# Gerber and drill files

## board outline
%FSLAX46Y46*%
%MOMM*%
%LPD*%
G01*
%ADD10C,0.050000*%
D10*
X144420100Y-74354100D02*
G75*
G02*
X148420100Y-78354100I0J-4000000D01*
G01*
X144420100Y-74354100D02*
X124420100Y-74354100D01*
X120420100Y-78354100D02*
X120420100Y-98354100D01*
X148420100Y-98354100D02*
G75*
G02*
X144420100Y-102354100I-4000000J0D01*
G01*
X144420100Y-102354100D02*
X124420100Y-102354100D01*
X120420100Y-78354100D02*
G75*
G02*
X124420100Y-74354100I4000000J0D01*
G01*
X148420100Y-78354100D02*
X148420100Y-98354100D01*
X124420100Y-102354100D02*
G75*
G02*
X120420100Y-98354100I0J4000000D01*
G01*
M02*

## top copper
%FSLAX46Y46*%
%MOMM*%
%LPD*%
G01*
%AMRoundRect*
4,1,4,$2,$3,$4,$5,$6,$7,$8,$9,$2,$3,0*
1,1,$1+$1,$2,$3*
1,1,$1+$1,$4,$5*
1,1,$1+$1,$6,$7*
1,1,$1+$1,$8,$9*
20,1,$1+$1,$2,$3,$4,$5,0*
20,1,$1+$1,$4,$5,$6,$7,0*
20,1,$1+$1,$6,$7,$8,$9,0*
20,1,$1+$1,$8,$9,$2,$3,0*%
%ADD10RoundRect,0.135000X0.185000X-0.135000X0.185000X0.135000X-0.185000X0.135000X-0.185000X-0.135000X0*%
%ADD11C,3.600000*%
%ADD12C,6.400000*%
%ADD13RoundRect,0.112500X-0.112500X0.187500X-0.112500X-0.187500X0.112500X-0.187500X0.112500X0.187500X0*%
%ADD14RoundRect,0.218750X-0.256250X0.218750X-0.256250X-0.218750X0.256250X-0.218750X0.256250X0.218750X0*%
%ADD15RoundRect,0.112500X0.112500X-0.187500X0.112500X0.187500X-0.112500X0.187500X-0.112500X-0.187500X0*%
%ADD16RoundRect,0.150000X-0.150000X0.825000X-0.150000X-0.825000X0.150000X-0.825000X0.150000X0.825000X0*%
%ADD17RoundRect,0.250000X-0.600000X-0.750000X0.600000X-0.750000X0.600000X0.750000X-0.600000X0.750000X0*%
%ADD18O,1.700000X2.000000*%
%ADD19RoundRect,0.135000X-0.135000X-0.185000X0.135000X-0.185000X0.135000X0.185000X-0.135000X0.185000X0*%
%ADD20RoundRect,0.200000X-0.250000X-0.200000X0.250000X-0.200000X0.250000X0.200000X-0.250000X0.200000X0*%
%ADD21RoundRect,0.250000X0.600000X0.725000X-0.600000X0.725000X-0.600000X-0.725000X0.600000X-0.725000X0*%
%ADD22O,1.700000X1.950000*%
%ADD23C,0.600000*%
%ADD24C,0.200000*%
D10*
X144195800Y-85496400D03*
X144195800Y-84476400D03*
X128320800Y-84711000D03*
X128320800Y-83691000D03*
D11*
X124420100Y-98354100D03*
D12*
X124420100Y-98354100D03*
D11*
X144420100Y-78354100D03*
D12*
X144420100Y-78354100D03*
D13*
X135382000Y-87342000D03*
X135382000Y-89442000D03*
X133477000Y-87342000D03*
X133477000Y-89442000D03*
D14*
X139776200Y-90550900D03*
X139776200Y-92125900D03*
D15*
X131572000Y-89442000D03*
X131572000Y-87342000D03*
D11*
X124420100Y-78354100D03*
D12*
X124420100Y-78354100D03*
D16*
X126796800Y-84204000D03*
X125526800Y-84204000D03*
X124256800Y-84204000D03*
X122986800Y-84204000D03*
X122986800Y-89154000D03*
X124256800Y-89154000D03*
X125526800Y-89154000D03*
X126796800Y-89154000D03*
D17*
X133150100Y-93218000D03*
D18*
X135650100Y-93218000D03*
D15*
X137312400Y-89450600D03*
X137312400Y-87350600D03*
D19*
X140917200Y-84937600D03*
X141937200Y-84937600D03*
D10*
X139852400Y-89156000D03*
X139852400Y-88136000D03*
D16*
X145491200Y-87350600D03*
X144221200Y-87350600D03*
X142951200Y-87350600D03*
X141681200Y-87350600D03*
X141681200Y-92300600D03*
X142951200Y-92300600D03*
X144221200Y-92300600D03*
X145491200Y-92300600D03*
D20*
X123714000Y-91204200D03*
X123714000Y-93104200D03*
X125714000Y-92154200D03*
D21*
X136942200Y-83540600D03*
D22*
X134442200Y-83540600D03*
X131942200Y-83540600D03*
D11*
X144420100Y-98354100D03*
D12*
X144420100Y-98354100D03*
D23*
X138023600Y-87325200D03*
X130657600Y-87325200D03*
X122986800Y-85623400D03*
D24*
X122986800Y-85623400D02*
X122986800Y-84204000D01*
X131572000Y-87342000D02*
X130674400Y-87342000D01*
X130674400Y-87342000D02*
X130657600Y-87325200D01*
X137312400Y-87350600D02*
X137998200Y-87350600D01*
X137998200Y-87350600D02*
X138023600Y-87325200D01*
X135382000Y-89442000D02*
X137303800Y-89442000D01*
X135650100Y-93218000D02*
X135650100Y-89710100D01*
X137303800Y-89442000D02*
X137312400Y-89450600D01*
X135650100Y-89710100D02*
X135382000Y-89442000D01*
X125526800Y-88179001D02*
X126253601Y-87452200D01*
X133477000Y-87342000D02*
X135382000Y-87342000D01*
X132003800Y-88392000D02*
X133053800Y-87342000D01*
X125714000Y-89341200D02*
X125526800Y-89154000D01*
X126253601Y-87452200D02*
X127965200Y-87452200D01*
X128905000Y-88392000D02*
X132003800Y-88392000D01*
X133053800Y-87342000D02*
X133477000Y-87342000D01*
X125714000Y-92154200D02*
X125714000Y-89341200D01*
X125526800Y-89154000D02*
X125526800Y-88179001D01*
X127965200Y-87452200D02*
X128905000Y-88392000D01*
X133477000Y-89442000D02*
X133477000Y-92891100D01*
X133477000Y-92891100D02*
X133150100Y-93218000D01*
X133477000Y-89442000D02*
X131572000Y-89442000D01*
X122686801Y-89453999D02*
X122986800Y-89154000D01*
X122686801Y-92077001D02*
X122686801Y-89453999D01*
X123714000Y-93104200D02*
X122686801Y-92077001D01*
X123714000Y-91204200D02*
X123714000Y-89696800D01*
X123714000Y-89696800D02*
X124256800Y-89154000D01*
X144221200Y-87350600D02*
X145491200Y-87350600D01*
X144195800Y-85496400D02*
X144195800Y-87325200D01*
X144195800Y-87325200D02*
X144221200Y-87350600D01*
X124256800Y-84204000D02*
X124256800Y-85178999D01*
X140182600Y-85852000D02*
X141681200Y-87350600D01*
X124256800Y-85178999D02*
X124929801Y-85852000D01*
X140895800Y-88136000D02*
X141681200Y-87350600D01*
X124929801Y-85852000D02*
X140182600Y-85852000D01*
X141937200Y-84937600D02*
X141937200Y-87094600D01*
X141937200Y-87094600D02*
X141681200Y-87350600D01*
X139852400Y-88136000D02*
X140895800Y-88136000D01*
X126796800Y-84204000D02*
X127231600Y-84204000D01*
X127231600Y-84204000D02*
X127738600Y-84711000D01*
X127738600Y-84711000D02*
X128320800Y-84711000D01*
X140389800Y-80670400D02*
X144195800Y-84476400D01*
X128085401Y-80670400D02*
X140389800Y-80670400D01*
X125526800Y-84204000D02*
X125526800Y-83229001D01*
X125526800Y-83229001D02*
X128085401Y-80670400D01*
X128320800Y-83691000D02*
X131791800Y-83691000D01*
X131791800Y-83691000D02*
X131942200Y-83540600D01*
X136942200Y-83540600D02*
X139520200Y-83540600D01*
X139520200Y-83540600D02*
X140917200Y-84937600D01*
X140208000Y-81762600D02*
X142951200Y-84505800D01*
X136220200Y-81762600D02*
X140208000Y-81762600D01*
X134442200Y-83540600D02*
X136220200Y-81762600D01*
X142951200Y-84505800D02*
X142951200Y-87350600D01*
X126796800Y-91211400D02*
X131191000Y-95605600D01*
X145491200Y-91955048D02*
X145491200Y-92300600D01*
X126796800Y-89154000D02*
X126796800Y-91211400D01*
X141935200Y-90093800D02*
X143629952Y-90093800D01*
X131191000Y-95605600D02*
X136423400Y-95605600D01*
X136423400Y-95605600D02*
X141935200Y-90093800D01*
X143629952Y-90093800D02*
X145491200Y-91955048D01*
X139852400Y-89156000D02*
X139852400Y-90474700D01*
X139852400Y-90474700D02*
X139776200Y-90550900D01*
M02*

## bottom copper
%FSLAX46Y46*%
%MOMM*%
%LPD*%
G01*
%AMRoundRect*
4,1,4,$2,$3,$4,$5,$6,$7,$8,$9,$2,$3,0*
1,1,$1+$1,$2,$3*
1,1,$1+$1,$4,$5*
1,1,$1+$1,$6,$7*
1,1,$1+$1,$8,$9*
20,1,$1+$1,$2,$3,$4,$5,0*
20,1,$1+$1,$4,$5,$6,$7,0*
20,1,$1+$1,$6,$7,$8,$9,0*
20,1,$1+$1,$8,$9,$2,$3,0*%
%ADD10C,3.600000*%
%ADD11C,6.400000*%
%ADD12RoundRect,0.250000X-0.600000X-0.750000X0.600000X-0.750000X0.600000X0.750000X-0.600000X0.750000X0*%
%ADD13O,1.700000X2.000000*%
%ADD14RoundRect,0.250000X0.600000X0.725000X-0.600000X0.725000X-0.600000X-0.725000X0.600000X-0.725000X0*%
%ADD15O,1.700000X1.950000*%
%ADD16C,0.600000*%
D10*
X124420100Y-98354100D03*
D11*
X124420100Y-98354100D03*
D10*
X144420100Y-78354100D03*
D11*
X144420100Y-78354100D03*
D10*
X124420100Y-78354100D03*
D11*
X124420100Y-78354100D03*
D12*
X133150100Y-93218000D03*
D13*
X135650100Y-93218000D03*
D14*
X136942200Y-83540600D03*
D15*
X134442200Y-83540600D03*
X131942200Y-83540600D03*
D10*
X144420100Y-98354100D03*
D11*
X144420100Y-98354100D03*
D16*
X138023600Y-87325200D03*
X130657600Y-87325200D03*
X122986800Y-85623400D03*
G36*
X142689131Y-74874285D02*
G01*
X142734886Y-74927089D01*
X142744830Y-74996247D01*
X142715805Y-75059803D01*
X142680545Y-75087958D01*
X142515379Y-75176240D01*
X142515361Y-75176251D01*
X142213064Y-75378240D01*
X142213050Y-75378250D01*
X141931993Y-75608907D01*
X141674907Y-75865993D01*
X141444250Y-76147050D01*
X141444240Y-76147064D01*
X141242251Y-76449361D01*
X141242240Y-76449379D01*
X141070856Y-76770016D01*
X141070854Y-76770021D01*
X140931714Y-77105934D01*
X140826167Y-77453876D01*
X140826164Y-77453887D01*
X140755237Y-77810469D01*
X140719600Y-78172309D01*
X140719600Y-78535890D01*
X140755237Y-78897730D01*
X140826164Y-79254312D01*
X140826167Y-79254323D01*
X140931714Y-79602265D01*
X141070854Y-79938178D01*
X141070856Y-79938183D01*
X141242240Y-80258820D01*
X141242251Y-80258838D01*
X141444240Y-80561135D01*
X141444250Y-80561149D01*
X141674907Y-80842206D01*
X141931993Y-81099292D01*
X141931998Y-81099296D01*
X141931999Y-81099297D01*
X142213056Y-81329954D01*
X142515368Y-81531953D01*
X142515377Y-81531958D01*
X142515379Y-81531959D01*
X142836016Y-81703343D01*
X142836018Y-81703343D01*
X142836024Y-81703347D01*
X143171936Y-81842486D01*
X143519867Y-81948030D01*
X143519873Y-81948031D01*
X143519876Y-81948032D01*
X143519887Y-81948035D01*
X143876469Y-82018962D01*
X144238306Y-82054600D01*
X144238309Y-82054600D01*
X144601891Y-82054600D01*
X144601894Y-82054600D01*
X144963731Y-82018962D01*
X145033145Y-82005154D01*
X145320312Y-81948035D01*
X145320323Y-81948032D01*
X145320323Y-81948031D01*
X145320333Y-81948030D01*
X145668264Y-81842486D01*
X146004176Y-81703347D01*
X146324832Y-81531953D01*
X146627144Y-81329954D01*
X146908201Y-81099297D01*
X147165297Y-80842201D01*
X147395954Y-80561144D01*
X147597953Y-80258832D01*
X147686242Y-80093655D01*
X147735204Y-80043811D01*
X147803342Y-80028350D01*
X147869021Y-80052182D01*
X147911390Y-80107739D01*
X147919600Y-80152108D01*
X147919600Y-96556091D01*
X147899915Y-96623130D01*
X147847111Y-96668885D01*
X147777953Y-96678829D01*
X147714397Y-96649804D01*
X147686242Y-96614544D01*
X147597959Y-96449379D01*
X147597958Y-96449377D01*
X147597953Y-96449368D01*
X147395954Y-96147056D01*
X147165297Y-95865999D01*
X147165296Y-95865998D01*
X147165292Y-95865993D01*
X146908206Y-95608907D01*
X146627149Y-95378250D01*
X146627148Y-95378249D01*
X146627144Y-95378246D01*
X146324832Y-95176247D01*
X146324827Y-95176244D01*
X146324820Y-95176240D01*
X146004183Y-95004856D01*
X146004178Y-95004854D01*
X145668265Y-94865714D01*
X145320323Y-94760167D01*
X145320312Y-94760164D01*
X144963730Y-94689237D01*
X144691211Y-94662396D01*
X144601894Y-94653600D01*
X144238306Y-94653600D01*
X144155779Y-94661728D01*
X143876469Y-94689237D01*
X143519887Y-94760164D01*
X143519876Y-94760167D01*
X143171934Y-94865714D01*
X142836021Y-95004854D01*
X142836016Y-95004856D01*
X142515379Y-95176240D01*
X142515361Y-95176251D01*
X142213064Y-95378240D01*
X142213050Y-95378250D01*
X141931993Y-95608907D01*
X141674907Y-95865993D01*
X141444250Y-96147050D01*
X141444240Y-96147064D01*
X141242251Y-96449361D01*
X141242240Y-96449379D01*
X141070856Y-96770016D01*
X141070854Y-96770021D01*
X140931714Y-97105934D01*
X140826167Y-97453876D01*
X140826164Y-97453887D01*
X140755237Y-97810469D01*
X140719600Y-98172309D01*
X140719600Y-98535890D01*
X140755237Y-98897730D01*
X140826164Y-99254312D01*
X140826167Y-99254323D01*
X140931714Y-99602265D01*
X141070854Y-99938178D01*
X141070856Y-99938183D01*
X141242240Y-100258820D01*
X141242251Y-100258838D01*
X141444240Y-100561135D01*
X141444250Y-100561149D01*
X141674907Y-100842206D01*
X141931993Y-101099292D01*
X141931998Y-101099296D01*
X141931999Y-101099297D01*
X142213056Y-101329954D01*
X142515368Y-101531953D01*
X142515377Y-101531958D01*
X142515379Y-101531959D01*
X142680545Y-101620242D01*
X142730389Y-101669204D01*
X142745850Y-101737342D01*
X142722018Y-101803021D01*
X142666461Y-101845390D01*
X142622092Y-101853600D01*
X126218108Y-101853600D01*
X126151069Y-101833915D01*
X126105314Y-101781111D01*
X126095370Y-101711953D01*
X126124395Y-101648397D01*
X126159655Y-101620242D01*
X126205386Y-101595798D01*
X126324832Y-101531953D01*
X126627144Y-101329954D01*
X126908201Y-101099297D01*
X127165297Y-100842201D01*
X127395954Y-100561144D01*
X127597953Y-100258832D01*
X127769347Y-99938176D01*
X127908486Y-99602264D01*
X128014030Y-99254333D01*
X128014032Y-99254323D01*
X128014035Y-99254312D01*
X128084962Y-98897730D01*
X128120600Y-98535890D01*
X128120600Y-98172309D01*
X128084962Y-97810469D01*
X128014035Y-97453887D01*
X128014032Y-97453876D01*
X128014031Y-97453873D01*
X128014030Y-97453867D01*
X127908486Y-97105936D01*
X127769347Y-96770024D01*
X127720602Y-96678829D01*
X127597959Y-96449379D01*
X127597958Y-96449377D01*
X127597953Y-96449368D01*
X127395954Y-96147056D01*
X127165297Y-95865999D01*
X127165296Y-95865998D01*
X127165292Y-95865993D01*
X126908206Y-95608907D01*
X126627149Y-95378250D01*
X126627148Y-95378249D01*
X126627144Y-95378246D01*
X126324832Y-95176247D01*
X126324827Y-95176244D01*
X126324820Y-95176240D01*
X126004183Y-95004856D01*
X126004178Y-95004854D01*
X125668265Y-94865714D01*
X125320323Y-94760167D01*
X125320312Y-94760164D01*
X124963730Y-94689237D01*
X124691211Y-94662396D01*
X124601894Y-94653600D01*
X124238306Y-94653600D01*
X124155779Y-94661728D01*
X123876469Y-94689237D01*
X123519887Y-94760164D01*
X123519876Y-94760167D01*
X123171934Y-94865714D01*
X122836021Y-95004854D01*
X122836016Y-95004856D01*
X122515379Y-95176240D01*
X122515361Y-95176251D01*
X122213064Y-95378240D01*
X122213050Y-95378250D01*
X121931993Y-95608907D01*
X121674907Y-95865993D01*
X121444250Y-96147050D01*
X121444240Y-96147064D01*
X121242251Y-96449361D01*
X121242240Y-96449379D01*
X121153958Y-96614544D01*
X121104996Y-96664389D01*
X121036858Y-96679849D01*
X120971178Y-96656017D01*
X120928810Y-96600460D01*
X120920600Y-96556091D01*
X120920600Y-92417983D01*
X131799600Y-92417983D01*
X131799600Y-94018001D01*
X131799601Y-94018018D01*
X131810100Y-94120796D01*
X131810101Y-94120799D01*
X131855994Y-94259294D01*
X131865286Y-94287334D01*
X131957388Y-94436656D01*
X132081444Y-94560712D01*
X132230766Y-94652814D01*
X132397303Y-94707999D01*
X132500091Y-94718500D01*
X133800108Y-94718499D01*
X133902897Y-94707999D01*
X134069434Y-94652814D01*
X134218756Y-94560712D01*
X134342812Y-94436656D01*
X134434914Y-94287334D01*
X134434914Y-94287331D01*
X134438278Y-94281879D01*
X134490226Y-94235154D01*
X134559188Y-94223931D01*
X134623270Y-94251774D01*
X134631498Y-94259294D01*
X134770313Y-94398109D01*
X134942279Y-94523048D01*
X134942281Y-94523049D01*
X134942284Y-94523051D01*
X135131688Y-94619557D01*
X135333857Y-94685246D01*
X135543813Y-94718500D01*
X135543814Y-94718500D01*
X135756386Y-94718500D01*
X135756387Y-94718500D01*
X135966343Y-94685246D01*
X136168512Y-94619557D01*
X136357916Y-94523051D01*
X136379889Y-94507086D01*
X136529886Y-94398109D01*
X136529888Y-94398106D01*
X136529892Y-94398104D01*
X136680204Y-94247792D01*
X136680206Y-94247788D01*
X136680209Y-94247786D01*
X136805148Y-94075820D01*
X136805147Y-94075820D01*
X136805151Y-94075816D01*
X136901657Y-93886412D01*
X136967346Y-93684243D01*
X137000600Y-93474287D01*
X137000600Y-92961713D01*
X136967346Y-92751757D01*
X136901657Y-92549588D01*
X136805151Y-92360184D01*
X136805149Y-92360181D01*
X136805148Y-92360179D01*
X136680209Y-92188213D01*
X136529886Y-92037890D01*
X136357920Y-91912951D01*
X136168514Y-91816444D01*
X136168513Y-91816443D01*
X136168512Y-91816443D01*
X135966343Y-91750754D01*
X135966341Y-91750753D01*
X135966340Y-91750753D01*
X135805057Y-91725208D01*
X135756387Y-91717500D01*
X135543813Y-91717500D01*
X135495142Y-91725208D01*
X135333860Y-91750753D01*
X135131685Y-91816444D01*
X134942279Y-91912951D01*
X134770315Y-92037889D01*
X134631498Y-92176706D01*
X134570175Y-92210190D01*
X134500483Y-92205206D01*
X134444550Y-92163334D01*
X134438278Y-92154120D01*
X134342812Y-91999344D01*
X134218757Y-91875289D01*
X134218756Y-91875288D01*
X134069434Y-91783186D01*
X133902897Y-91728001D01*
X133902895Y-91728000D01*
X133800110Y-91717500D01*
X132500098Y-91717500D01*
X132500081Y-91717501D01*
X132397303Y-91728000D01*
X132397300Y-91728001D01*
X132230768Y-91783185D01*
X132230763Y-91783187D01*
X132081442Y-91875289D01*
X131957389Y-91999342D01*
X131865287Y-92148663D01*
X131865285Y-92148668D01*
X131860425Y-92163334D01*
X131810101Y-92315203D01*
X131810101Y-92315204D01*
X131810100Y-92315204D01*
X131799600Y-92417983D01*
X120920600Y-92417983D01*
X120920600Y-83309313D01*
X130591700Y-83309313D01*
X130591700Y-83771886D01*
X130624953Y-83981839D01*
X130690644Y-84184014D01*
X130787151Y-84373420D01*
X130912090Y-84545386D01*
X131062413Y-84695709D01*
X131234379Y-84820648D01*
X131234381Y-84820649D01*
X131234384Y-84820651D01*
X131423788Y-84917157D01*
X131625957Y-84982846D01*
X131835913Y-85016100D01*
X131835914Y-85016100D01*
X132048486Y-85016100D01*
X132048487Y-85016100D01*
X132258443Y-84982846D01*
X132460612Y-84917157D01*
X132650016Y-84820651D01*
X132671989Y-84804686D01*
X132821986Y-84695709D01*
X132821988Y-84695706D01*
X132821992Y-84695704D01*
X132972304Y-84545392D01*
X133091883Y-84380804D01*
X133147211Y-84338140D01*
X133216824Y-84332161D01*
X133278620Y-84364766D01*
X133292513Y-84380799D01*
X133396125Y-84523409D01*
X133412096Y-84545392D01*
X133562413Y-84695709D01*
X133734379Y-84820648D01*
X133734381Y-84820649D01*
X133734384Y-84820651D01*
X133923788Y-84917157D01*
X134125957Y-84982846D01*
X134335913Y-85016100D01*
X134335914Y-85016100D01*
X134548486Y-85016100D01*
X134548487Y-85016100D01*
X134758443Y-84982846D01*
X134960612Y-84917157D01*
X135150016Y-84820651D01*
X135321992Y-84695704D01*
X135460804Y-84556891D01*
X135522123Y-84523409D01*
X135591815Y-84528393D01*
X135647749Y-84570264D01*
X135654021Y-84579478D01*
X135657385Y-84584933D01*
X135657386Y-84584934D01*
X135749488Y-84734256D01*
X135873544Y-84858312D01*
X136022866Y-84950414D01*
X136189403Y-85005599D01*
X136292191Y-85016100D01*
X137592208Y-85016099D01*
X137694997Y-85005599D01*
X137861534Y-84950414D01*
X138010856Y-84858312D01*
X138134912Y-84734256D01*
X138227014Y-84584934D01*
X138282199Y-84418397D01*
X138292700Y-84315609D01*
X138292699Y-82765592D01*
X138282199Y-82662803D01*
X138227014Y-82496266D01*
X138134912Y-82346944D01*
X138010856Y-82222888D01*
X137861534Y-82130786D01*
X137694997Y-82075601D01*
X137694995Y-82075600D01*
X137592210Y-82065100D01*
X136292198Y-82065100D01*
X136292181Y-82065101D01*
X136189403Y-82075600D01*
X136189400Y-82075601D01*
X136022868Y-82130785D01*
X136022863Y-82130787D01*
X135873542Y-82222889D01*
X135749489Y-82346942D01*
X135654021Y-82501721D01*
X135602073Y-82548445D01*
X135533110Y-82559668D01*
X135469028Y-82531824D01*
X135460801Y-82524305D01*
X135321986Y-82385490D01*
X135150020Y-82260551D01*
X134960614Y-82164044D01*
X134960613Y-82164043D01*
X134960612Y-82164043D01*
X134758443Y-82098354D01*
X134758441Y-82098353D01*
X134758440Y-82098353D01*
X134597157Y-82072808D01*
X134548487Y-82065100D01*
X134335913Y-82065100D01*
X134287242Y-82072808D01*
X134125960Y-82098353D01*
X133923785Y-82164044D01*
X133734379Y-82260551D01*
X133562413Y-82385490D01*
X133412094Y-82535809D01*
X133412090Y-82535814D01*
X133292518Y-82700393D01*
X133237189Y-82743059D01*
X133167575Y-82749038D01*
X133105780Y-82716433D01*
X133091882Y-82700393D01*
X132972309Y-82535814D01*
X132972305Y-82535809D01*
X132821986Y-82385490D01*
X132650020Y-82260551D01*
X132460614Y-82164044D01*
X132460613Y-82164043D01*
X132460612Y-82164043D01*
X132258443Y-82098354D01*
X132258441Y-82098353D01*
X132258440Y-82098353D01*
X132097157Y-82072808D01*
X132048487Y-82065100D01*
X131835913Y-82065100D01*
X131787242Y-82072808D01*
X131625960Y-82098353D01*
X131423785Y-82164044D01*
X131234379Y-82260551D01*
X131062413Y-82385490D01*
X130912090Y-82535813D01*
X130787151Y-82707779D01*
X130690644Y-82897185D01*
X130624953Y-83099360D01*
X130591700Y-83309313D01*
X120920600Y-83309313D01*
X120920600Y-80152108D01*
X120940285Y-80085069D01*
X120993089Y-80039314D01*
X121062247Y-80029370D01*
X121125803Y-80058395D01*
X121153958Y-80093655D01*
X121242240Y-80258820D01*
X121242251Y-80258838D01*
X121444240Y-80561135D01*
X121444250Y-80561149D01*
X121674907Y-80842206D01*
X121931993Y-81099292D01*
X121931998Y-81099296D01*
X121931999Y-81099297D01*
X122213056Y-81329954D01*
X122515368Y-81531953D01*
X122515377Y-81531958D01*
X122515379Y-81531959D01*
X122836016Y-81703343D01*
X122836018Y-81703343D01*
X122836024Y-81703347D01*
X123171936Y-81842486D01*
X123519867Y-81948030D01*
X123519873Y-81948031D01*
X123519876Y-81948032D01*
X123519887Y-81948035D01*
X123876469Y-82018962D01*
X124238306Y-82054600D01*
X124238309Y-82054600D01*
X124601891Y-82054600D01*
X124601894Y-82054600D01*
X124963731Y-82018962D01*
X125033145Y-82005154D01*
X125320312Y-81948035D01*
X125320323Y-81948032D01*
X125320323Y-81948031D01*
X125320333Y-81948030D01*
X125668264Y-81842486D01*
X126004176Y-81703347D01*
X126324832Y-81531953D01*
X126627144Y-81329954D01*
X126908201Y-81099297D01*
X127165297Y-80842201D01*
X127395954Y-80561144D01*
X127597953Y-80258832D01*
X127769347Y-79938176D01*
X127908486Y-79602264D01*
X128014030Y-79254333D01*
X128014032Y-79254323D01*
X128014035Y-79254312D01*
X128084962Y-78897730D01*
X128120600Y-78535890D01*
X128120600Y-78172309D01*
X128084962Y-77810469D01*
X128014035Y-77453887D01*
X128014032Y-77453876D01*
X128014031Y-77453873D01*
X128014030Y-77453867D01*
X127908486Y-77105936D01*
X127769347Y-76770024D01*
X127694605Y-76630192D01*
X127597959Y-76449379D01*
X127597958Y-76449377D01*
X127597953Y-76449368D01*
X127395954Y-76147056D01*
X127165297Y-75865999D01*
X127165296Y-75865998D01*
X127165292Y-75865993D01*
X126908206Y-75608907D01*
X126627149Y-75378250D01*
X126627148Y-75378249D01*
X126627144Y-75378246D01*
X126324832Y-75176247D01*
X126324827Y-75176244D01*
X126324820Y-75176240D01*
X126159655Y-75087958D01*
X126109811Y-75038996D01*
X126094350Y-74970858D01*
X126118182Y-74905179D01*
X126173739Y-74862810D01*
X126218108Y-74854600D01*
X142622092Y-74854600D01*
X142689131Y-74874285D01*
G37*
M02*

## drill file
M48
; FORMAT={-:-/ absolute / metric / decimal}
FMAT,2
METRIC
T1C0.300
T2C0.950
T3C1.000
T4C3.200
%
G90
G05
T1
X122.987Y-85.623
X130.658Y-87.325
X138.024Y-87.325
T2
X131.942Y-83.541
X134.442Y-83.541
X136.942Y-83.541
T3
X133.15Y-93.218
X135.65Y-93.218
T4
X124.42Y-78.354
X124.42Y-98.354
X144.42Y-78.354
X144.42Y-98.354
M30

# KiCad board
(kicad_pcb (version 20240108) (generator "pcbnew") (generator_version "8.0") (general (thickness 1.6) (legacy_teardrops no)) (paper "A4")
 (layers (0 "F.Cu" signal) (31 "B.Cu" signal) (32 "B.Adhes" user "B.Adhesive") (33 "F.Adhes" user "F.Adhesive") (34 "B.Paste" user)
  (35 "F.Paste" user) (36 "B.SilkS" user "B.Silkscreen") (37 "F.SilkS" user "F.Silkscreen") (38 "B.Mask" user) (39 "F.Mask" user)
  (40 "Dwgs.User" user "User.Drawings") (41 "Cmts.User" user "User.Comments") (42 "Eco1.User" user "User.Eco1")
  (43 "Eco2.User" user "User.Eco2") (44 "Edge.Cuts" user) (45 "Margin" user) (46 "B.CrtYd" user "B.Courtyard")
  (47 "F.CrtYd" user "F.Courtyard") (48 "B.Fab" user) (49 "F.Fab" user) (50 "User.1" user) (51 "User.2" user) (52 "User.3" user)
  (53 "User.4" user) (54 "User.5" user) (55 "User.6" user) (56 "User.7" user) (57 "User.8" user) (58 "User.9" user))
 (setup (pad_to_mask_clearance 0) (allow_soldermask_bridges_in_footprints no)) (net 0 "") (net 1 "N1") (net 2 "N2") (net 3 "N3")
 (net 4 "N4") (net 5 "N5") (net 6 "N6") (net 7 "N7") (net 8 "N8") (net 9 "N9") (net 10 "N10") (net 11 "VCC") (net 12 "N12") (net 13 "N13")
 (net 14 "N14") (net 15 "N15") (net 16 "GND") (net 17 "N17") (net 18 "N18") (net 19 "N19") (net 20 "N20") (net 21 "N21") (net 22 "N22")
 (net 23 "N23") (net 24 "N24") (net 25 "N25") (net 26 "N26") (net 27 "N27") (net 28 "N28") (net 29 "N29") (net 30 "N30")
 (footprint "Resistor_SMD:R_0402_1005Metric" (layer "F.Cu") (at 144.1958 84.9864 90)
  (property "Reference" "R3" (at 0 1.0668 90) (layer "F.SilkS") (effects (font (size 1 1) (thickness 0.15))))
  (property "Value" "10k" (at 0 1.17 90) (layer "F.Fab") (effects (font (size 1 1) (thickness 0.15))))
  (pad "1" smd roundrect (at -0.51 0 90) (size 0.54 0.64) (layers "F.Cu" "F.Paste" "F.Mask") (roundrect_rratio 0.25) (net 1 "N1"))
  (pad "2" smd roundrect (at 0.51 0 90) (size 0.54 0.64) (layers "F.Cu" "F.Paste" "F.Mask") (roundrect_rratio 0.25) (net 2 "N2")))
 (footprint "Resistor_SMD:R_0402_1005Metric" (layer "F.Cu") (at 128.3208 84.201 90)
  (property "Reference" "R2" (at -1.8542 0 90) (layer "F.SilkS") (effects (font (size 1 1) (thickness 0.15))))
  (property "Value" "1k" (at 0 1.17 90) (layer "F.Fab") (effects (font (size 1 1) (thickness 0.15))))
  (pad "1" smd roundrect (at -0.51 0 90) (size 0.54 0.64) (layers "F.Cu" "F.Paste" "F.Mask") (roundrect_rratio 0.25) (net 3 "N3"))
  (pad "2" smd roundrect (at 0.51 0 90) (size 0.54 0.64) (layers "F.Cu" "F.Paste" "F.Mask") (roundrect_rratio 0.25) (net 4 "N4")))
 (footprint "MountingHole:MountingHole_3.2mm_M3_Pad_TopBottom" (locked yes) (layer "F.Cu") (at 124.4201 98.3541)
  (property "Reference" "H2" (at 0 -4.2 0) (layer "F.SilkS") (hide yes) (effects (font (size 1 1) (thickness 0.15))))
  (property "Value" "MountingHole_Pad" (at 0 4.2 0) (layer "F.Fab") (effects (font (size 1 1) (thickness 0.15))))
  (pad "1" thru_hole circle (at 0 0) (size 3.6 3.6) (drill 3.2) (layers "*.Cu" "*.Mask") (remove_unused_layers no) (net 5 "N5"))
  (pad "1" connect circle (at 0 0) (size 6.4 6.4) (layers "F.Cu" "F.Mask") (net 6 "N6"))
  (pad "1" connect circle (at 0 0) (size 6.4 6.4) (layers "B.Cu" "B.Mask") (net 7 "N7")))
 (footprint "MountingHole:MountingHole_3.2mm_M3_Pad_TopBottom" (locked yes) (layer "F.Cu") (at 144.4201 78.3541)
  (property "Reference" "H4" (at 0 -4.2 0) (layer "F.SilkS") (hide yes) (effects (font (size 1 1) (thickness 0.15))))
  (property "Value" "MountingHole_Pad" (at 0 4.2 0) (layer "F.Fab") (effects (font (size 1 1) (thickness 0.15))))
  (pad "1" thru_hole circle (at 0 0) (size 3.6 3.6) (drill 3.2) (layers "*.Cu" "*.Mask") (remove_unused_layers no) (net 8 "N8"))
  (pad "1" connect circle (at 0 0) (size 6.4 6.4) (layers "F.Cu" "F.Mask") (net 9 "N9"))
  (pad "1" connect circle (at 0 0) (size 6.4 6.4) (layers "B.Cu" "B.Mask") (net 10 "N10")))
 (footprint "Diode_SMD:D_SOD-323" (layer "F.Cu") (at 135.382 88.392 -90)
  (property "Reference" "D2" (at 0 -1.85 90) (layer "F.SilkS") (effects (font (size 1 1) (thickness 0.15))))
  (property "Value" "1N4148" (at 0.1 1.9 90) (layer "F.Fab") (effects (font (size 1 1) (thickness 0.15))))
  (pad "1" smd roundrect (at -1.05 0 270) (size 0.6 0.45) (layers "F.Cu" "F.Paste" "F.Mask") (roundrect_rratio 0.25) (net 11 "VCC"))
  (pad "2" smd roundrect (at 1.05 0 270) (size 0.6 0.45) (layers "F.Cu" "F.Paste" "F.Mask") (roundrect_rratio 0.25) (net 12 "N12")))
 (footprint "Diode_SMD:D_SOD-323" (layer "F.Cu") (at 133.477 88.392 -90)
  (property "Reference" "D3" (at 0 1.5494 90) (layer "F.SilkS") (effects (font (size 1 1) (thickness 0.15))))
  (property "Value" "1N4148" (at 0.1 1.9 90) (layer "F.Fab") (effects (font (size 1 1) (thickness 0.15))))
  (pad "1" smd roundrect (at -1.05 0 270) (size 0.6 0.45) (layers "F.Cu" "F.Paste" "F.Mask") (roundrect_rratio 0.25) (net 11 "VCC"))
  (pad "2" smd roundrect (at 1.05 0 270) (size 0.6 0.45) (layers "F.Cu" "F.Paste" "F.Mask") (roundrect_rratio 0.25) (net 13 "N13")))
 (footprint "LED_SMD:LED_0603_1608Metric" (layer "F.Cu") (at 139.7762 91.3384 -90)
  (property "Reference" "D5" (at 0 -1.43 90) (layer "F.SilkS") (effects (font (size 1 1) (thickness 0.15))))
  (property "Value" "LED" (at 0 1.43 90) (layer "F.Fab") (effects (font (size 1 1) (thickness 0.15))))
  (pad "1" smd roundrect (at -0.7875 0 270) (size 0.875 0.95) (layers "F.Cu" "F.Paste" "F.Mask") (roundrect_rratio 0.25) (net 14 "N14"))
  (pad "2" smd roundrect (at 0.7875 0 270) (size 0.875 0.95) (layers "F.Cu" "F.Paste" "F.Mask") (roundrect_rratio 0.25) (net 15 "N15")))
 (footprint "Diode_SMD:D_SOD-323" (layer "F.Cu") (at 131.572 88.392 90)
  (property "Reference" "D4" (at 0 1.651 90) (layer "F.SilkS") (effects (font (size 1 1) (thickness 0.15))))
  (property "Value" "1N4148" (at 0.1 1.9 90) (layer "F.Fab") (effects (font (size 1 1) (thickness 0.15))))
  (pad "1" smd roundrect (at -1.05 0 90) (size 0.6 0.45) (layers "F.Cu" "F.Paste" "F.Mask") (roundrect_rratio 0.25) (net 13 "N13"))
  (pad "2" smd roundrect (at 1.05 0 90) (size 0.6 0.45) (layers "F.Cu" "F.Paste" "F.Mask") (roundrect_rratio 0.25) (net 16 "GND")))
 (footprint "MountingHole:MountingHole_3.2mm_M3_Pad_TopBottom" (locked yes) (layer "F.Cu") (at 124.4201 78.3541)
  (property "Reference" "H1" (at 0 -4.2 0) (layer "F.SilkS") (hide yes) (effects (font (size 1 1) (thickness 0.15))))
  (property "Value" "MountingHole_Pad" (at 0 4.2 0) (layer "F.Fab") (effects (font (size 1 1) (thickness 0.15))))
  (pad "1" thru_hole circle (at 0 0) (size 3.6 3.6) (drill 3.2) (layers "*.Cu" "*.Mask") (remove_unused_layers no) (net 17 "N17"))
  (pad "1" connect circle (at 0 0) (size 6.4 6.4) (layers "F.Cu" "F.Mask") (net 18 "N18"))
  (pad "1" connect circle (at 0 0) (size 6.4 6.4) (layers "B.Cu" "B.Mask") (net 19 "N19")))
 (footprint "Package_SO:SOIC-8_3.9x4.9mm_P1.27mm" (layer "F.Cu") (at 124.8918 86.679 -90)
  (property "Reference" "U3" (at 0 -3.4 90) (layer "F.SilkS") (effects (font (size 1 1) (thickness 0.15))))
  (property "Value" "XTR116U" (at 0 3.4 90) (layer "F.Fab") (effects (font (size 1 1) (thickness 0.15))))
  (pad "1" smd roundrect (at -2.475 -1.905 270) (size 1.95 0.6) (layers "F.Cu" "F.Paste" "F.Mask") (roundrect_rratio 0.25) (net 3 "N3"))
  (pad "2" smd roundrect (at -2.475 -0.635 270) (size 1.95 0.6) (layers "F.Cu" "F.Paste" "F.Mask") (roundrect_rratio 0.25) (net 2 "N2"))
  (pad "3" smd roundrect (at -2.475 0.635 270) (size 1.95 0.6) (layers "F.Cu" "F.Paste" "F.Mask") (roundrect_rratio 0.25) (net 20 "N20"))
  (pad "4" smd roundrect (at -2.475 1.905 270) (size 1.95 0.6) (layers "F.Cu" "F.Paste" "F.Mask") (roundrect_rratio 0.25) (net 16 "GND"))
  (pad "5" smd roundrect (at 2.475 1.905 270) (size 1.95 0.6) (layers "F.Cu" "F.Paste" "F.Mask") (roundrect_rratio 0.25) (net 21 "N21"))
  (pad "6" smd roundrect (at 2.475 0.635 270) (size 1.95 0.6) (layers "F.Cu" "F.Paste" "F.Mask") (roundrect_rratio 0.25) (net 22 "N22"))
  (pad "7" smd roundrect (at 2.475 -0.635 270) (size 1.95 0.6) (layers "F.Cu" "F.Paste" "F.Mask") (roundrect_rratio 0.25) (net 11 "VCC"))
  (pad "8" smd roundrect (at 2.475 -1.905 270) (size 1.95 0.6) (layers "F.Cu" "F.Paste" "F.Mask") (roundrect_rratio 0.25) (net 15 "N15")))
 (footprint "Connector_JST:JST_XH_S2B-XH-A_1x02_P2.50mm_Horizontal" (layer "F.Cu") (at 133.1501 93.218)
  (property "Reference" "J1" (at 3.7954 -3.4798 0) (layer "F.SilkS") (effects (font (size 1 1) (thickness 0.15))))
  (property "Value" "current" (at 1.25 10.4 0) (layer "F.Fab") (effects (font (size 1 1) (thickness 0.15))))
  (pad "1" thru_hole roundrect (at 0 0) (size 1.7 2) (drill 1) (layers "*.Cu" "*.Mask") (remove_unused_layers no)
   (roundrect_rratio 0.147059) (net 13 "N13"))
  (pad "2" thru_hole oval (at 2.5 0) (size 1.7 2) (drill 1) (layers "*.Cu" "*.Mask") (remove_unused_layers no) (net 12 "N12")))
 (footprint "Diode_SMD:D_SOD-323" (layer "F.Cu") (at 137.3124 88.4006 90)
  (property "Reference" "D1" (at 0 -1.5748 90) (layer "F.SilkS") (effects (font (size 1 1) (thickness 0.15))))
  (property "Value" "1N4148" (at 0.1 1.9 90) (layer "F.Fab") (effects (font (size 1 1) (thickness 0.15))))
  (pad "1" smd roundrect (at -1.05 0 90) (size 0.6 0.45) (layers "F.Cu" "F.Paste" "F.Mask") (roundrect_rratio 0.25) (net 12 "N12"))
  (pad "2" smd roundrect (at 1.05 0 90) (size 0.6 0.45) (layers "F.Cu" "F.Paste" "F.Mask") (roundrect_rratio 0.25) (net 16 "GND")))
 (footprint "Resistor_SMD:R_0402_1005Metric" (layer "F.Cu") (at 141.4272 84.9376)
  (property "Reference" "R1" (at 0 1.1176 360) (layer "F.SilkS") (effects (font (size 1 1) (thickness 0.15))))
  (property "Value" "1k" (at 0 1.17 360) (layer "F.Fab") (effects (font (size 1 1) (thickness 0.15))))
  (pad "1" smd roundrect (at -0.51 0) (size 0.54 0.64) (layers "F.Cu" "F.Paste" "F.Mask") (roundrect_rratio 0.25) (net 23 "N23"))
  (pad "2" smd roundrect (at 0.51 0) (size 0.54 0.64) (layers "F.Cu" "F.Paste" "F.Mask") (roundrect_rratio 0.25) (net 20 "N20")))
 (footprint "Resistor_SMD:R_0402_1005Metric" (layer "F.Cu") (at 139.8524 88.646 90)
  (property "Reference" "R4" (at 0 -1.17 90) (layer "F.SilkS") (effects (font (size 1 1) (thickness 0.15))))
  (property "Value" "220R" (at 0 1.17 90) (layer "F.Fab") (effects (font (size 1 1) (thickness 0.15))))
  (pad "1" smd roundrect (at -0.51 0 90) (size 0.54 0.64) (layers "F.Cu" "F.Paste" "F.Mask") (roundrect_rratio 0.25) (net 14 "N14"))
  (pad "2" smd roundrect (at 0.51 0 90) (size 0.54 0.64) (layers "F.Cu" "F.Paste" "F.Mask") (roundrect_rratio 0.25) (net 20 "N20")))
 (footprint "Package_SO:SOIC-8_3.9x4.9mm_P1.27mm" (layer "F.Cu") (at 143.5862 89.8256 -90)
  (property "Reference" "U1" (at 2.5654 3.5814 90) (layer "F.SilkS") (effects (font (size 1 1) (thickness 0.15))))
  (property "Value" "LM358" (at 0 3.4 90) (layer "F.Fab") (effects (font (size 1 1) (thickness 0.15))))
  (pad "1" smd roundrect (at -2.475 -1.905 270) (size 1.95 0.6) (layers "F.Cu" "F.Paste" "F.Mask") (roundrect_rratio 0.25) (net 1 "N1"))
  (pad "2" smd roundrect (at -2.475 -0.635 270) (size 1.95 0.6) (layers "F.Cu" "F.Paste" "F.Mask") (roundrect_rratio 0.25) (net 1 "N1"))
  (pad "3" smd roundrect (at -2.475 0.635 270) (size 1.95 0.6) (layers "F.Cu" "F.Paste" "F.Mask") (roundrect_rratio 0.25) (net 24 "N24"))
  (pad "4" smd roundrect (at -2.475 1.905 270) (size 1.95 0.6) (layers "F.Cu" "F.Paste" "F.Mask") (roundrect_rratio 0.25) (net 20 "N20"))
  (pad "5" smd roundrect (at 2.475 1.905 270) (size 1.95 0.6) (layers "F.Cu" "F.Paste" "F.Mask") (roundrect_rratio 0.25) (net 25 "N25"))
  (pad "6" smd roundrect (at 2.475 0.635 270) (size 1.95 0.6) (layers "F.Cu" "F.Paste" "F.Mask") (roundrect_rratio 0.25) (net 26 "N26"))
  (pad "7" smd roundrect (at 2.475 -0.635 270) (size 1.95 0.6) (layers "F.Cu" "F.Paste" "F.Mask") (roundrect_rratio 0.25) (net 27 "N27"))
  (pad "8" smd roundrect (at 2.475 -1.905 270) (size 1.95 0.6) (layers "F.Cu" "F.Paste" "F.Mask") (roundrect_rratio 0.25) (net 15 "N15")))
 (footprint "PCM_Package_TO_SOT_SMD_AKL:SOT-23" (layer "F.Cu") (at 124.714 92.1542)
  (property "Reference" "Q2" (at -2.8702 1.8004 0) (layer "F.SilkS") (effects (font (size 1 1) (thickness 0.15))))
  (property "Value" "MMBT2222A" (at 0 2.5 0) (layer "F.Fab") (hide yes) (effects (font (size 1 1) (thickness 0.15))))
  (pad "1" smd roundrect (at -1 -0.95) (size 0.9 0.8) (layers "F.Cu" "F.Paste" "F.Mask") (roundrect_rratio 0.25) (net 22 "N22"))
  (pad "2" smd roundrect (at -1 0.95) (size 0.9 0.8) (layers "F.Cu" "F.Paste" "F.Mask") (roundrect_rratio 0.25) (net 21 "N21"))
  (pad "3" smd roundrect (at 1 0) (size 0.9 0.8) (layers "F.Cu" "F.Paste" "F.Mask") (roundrect_rratio 0.25) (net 11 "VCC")))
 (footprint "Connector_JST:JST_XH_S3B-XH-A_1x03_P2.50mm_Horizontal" (layer "F.Cu") (at 136.9422 83.5406 180)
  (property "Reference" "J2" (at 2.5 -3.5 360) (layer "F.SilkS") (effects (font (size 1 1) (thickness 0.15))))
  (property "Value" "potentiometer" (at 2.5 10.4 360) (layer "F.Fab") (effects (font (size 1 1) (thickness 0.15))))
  (pad "1" thru_hole roundrect (at 0 0 180) (size 1.7 1.95) (drill 0.95) (layers "*.Cu" "*.Mask") (remove_unused_layers no)
   (roundrect_rratio 0.147059) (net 23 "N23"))
  (pad "2" thru_hole oval (at 2.5 0 180) (size 1.7 1.95) (drill 0.95) (layers "*.Cu" "*.Mask") (remove_unused_layers no) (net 24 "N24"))
  (pad "3" thru_hole oval (at 5 0 180) (size 1.7 1.95) (drill 0.95) (layers "*.Cu" "*.Mask") (remove_unused_layers no) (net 4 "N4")))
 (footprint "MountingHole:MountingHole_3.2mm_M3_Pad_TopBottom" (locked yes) (layer "F.Cu") (at 144.4201 98.3541)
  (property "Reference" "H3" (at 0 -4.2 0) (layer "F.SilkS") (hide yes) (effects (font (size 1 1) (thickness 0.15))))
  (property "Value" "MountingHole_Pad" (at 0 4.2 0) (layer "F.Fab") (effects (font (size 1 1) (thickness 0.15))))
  (pad "1" thru_hole circle (at 0 0) (size 3.6 3.6) (drill 3.2) (layers "*.Cu" "*.Mask") (remove_unused_layers no) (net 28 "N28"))
  (pad "1" connect circle (at 0 0) (size 6.4 6.4) (layers "F.Cu" "F.Mask") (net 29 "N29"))
  (pad "1" connect circle (at 0 0) (size 6.4 6.4) (layers "B.Cu" "B.Mask") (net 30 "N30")))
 (gr_arc (start 144.4201 74.3541) (mid 147.248527 75.525673) (end 148.4201 78.3541) (stroke (width 0.05) (type default)) (layer "Edge.Cuts"))
 (gr_line (start 144.4201 74.3541) (end 124.4201 74.3541) (stroke (width 0.05) (type default)) (layer "Edge.Cuts"))
 (gr_line (start 120.4201 78.3541) (end 120.4201 98.3541) (stroke (width 0.05) (type default)) (layer "Edge.Cuts"))
 (gr_arc (start 148.4201 98.3541) (mid 147.248527 101.182527) (end 144.4201 102.3541) (stroke (width 0.05) (type default))
  (layer "Edge.Cuts"))
 (gr_line (start 144.4201 102.3541) (end 124.4201 102.3541) (stroke (width 0.05) (type default)) (layer "Edge.Cuts"))
 (gr_arc (start 120.4201 78.3541) (mid 121.591673 75.525673) (end 124.4201 74.3541) (stroke (width 0.05) (type default)) (layer "Edge.Cuts"))
 (gr_line (start 148.4201 78.3541) (end 148.4201 98.3541) (stroke (width 0.05) (type default)) (layer "Edge.Cuts"))
 (gr_arc (start 124.4201 102.3541) (mid 121.591673 101.182527) (end 120.4201 98.3541) (stroke (width 0.05) (type default))
  (layer "Edge.Cuts"))
 (segment (start 122.9868 85.6234) (end 122.9868 84.204) (width 0.2) (layer "F.Cu") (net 16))
 (segment (start 131.572 87.342) (end 130.6744 87.342) (width 0.2) (layer "F.Cu") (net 16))
 (segment (start 130.6744 87.342) (end 130.6576 87.3252) (width 0.2) (layer "F.Cu") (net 16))
 (segment (start 137.3124 87.3506) (end 137.9982 87.3506) (width 0.2) (layer "F.Cu") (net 16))
 (segment (start 137.9982 87.3506) (end 138.0236 87.3252) (width 0.2) (layer "F.Cu") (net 16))
 (via (at 138.0236 87.3252) (size 0.6) (drill 0.3) (layers "F.Cu" "B.Cu") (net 16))
 (via (at 130.6576 87.3252) (size 0.6) (drill 0.3) (layers "F.Cu" "B.Cu") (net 16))
 (via (at 122.9868 85.6234) (size 0.6) (drill 0.3) (layers "F.Cu" "B.Cu") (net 16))
 (segment (start 135.382 89.442) (end 137.3038 89.442) (width 0.2) (layer "F.Cu") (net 12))
 (segment (start 135.6501 93.218) (end 135.6501 89.7101) (width 0.2) (layer "F.Cu") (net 12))
 (segment (start 137.3038 89.442) (end 137.3124 89.4506) (width 0.2) (layer "F.Cu") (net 12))
 (segment (start 135.6501 89.7101) (end 135.382 89.442) (width 0.2) (layer "F.Cu") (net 12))
 (segment (start 125.5268 88.179001) (end 126.253601 87.4522) (width 0.2) (layer "F.Cu") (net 11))
 (segment (start 133.477 87.342) (end 135.382 87.342) (width 0.2) (layer "F.Cu") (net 11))
 (segment (start 132.0038 88.392) (end 133.0538 87.342) (width 0.2) (layer "F.Cu") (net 11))
 (segment (start 125.714 89.3412) (end 125.5268 89.154) (width 0.2) (layer "F.Cu") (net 11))
 (segment (start 126.253601 87.4522) (end 127.9652 87.4522) (width 0.2) (layer "F.Cu") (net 11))
 (segment (start 128.905 88.392) (end 132.0038 88.392) (width 0.2) (layer "F.Cu") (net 11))
 (segment (start 133.0538 87.342) (end 133.477 87.342) (width 0.2) (layer "F.Cu") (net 11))
 (segment (start 125.714 92.1542) (end 125.714 89.3412) (width 0.2) (layer "F.Cu") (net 11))
 (segment (start 125.5268 89.154) (end 125.5268 88.179001) (width 0.2) (layer "F.Cu") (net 11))
 (segment (start 127.9652 87.4522) (end 128.905 88.392) (width 0.2) (layer "F.Cu") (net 11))
 (segment (start 133.477 89.442) (end 133.477 92.8911) (width 0.2) (layer "F.Cu") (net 13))
 (segment (start 133.477 92.8911) (end 133.1501 93.218) (width 0.2) (layer "F.Cu") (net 13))
 (segment (start 133.477 89.442) (end 131.572 89.442) (width 0.2) (layer "F.Cu") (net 13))
 (segment (start 122.686801 89.453999) (end 122.9868 89.154) (width 0.2) (layer "F.Cu") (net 21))
 (segment (start 122.686801 92.077001) (end 122.686801 89.453999) (width 0.2) (layer "F.Cu") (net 21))
 (segment (start 123.714 93.1042) (end 122.686801 92.077001) (width 0.2) (layer "F.Cu") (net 21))
 (segment (start 123.714 91.2042) (end 123.714 89.6968) (width 0.2) (layer "F.Cu") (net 22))
 (segment (start 123.714 89.6968) (end 124.2568 89.154) (width 0.2) (layer "F.Cu") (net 22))
 (segment (start 144.2212 87.3506) (end 145.4912 87.3506) (width 0.2) (layer "F.Cu") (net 1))
 (segment (start 144.1958 85.4964) (end 144.1958 87.3252) (width 0.2) (layer "F.Cu") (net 1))
 (segment (start 144.1958 87.3252) (end 144.2212 87.3506) (width 0.2) (layer "F.Cu") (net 1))
 (segment (start 124.2568 84.204) (end 124.2568 85.178999) (width 0.2) (layer "F.Cu") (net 20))
 (segment (start 140.1826 85.852) (end 141.6812 87.3506) (width 0.2) (layer "F.Cu") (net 20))
 (segment (start 124.2568 85.178999) (end 124.929801 85.852) (width 0.2) (layer "F.Cu") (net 20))
 (segment (start 140.8958 88.136) (end 141.6812 87.3506) (width 0.2) (layer "F.Cu") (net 20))
 (segment (start 124.929801 85.852) (end 140.1826 85.852) (width 0.2) (layer "F.Cu") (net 20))
 (segment (start 141.9372 84.9376) (end 141.9372 87.0946) (width 0.2) (layer "F.Cu") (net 20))
 (segment (start 141.9372 87.0946) (end 141.6812 87.3506) (width 0.2) (layer "F.Cu") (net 20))
 (segment (start 139.8524 88.136) (end 140.8958 88.136) (width 0.2) (layer "F.Cu") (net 20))
 (segment (start 126.7968 84.204) (end 127.2316 84.204) (width 0.2) (layer "F.Cu") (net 3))
 (segment (start 127.2316 84.204) (end 127.7386 84.711) (width 0.2) (layer "F.Cu") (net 3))
 (segment (start 127.7386 84.711) (end 128.3208 84.711) (width 0.2) (layer "F.Cu") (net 3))
 (segment (start 140.3898 80.6704) (end 144.1958 84.4764) (width 0.2) (layer "F.Cu") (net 2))
 (segment (start 128.085401 80.6704) (end 140.3898 80.6704) (width 0.2) (layer "F.Cu") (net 2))
 (segment (start 125.5268 84.204) (end 125.5268 83.229001) (width 0.2) (layer "F.Cu") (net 2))
 (segment (start 125.5268 83.229001) (end 128.085401 80.6704) (width 0.2) (layer "F.Cu") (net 2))
 (segment (start 128.3208 83.691) (end 131.7918 83.691) (width 0.2) (layer "F.Cu") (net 4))
 (segment (start 131.7918 83.691) (end 131.9422 83.5406) (width 0.2) (layer "F.Cu") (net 4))
 (segment (start 136.9422 83.5406) (end 139.5202 83.5406) (width 0.2) (layer "F.Cu") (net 23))
 (segment (start 139.5202 83.5406) (end 140.9172 84.9376) (width 0.2) (layer "F.Cu") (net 23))
 (segment (start 140.208 81.7626) (end 142.9512 84.5058) (width 0.2) (layer "F.Cu") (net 24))
 (segment (start 136.2202 81.7626) (end 140.208 81.7626) (width 0.2) (layer "F.Cu") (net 24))
 (segment (start 134.4422 83.5406) (end 136.2202 81.7626) (width 0.2) (layer "F.Cu") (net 24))
 (segment (start 142.9512 84.5058) (end 142.9512 87.3506) (width 0.2) (layer "F.Cu") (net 24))
 (segment (start 126.7968 91.2114) (end 131.191 95.6056) (width 0.2) (layer "F.Cu") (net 15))
 (segment (start 145.4912 91.955048) (end 145.4912 92.3006) (width 0.2) (layer "F.Cu") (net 15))
 (segment (start 126.7968 89.154) (end 126.7968 91.2114) (width 0.2) (layer "F.Cu") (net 15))
 (segment (start 141.9352 90.0938) (end 143.629952 90.0938) (width 0.2) (layer "F.Cu") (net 15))
 (segment (start 131.191 95.6056) (end 136.4234 95.6056) (width 0.2) (layer "F.Cu") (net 15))
 (segment (start 136.4234 95.6056) (end 141.9352 90.0938) (width 0.2) (layer "F.Cu") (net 15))
 (segment (start 143.629952 90.0938) (end 145.4912 91.955048) (width 0.2) (layer "F.Cu") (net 15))
 (segment (start 139.8524 89.156) (end 139.8524 90.4747) (width 0.2) (layer "F.Cu") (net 14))
 (segment (start 139.8524 90.4747) (end 139.7762 90.5509) (width 0.2) (layer "F.Cu") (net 14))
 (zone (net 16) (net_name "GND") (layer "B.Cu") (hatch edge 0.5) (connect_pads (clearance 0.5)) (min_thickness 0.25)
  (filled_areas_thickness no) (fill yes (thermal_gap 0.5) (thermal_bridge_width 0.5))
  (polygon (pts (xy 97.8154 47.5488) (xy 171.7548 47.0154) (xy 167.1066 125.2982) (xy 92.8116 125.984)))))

